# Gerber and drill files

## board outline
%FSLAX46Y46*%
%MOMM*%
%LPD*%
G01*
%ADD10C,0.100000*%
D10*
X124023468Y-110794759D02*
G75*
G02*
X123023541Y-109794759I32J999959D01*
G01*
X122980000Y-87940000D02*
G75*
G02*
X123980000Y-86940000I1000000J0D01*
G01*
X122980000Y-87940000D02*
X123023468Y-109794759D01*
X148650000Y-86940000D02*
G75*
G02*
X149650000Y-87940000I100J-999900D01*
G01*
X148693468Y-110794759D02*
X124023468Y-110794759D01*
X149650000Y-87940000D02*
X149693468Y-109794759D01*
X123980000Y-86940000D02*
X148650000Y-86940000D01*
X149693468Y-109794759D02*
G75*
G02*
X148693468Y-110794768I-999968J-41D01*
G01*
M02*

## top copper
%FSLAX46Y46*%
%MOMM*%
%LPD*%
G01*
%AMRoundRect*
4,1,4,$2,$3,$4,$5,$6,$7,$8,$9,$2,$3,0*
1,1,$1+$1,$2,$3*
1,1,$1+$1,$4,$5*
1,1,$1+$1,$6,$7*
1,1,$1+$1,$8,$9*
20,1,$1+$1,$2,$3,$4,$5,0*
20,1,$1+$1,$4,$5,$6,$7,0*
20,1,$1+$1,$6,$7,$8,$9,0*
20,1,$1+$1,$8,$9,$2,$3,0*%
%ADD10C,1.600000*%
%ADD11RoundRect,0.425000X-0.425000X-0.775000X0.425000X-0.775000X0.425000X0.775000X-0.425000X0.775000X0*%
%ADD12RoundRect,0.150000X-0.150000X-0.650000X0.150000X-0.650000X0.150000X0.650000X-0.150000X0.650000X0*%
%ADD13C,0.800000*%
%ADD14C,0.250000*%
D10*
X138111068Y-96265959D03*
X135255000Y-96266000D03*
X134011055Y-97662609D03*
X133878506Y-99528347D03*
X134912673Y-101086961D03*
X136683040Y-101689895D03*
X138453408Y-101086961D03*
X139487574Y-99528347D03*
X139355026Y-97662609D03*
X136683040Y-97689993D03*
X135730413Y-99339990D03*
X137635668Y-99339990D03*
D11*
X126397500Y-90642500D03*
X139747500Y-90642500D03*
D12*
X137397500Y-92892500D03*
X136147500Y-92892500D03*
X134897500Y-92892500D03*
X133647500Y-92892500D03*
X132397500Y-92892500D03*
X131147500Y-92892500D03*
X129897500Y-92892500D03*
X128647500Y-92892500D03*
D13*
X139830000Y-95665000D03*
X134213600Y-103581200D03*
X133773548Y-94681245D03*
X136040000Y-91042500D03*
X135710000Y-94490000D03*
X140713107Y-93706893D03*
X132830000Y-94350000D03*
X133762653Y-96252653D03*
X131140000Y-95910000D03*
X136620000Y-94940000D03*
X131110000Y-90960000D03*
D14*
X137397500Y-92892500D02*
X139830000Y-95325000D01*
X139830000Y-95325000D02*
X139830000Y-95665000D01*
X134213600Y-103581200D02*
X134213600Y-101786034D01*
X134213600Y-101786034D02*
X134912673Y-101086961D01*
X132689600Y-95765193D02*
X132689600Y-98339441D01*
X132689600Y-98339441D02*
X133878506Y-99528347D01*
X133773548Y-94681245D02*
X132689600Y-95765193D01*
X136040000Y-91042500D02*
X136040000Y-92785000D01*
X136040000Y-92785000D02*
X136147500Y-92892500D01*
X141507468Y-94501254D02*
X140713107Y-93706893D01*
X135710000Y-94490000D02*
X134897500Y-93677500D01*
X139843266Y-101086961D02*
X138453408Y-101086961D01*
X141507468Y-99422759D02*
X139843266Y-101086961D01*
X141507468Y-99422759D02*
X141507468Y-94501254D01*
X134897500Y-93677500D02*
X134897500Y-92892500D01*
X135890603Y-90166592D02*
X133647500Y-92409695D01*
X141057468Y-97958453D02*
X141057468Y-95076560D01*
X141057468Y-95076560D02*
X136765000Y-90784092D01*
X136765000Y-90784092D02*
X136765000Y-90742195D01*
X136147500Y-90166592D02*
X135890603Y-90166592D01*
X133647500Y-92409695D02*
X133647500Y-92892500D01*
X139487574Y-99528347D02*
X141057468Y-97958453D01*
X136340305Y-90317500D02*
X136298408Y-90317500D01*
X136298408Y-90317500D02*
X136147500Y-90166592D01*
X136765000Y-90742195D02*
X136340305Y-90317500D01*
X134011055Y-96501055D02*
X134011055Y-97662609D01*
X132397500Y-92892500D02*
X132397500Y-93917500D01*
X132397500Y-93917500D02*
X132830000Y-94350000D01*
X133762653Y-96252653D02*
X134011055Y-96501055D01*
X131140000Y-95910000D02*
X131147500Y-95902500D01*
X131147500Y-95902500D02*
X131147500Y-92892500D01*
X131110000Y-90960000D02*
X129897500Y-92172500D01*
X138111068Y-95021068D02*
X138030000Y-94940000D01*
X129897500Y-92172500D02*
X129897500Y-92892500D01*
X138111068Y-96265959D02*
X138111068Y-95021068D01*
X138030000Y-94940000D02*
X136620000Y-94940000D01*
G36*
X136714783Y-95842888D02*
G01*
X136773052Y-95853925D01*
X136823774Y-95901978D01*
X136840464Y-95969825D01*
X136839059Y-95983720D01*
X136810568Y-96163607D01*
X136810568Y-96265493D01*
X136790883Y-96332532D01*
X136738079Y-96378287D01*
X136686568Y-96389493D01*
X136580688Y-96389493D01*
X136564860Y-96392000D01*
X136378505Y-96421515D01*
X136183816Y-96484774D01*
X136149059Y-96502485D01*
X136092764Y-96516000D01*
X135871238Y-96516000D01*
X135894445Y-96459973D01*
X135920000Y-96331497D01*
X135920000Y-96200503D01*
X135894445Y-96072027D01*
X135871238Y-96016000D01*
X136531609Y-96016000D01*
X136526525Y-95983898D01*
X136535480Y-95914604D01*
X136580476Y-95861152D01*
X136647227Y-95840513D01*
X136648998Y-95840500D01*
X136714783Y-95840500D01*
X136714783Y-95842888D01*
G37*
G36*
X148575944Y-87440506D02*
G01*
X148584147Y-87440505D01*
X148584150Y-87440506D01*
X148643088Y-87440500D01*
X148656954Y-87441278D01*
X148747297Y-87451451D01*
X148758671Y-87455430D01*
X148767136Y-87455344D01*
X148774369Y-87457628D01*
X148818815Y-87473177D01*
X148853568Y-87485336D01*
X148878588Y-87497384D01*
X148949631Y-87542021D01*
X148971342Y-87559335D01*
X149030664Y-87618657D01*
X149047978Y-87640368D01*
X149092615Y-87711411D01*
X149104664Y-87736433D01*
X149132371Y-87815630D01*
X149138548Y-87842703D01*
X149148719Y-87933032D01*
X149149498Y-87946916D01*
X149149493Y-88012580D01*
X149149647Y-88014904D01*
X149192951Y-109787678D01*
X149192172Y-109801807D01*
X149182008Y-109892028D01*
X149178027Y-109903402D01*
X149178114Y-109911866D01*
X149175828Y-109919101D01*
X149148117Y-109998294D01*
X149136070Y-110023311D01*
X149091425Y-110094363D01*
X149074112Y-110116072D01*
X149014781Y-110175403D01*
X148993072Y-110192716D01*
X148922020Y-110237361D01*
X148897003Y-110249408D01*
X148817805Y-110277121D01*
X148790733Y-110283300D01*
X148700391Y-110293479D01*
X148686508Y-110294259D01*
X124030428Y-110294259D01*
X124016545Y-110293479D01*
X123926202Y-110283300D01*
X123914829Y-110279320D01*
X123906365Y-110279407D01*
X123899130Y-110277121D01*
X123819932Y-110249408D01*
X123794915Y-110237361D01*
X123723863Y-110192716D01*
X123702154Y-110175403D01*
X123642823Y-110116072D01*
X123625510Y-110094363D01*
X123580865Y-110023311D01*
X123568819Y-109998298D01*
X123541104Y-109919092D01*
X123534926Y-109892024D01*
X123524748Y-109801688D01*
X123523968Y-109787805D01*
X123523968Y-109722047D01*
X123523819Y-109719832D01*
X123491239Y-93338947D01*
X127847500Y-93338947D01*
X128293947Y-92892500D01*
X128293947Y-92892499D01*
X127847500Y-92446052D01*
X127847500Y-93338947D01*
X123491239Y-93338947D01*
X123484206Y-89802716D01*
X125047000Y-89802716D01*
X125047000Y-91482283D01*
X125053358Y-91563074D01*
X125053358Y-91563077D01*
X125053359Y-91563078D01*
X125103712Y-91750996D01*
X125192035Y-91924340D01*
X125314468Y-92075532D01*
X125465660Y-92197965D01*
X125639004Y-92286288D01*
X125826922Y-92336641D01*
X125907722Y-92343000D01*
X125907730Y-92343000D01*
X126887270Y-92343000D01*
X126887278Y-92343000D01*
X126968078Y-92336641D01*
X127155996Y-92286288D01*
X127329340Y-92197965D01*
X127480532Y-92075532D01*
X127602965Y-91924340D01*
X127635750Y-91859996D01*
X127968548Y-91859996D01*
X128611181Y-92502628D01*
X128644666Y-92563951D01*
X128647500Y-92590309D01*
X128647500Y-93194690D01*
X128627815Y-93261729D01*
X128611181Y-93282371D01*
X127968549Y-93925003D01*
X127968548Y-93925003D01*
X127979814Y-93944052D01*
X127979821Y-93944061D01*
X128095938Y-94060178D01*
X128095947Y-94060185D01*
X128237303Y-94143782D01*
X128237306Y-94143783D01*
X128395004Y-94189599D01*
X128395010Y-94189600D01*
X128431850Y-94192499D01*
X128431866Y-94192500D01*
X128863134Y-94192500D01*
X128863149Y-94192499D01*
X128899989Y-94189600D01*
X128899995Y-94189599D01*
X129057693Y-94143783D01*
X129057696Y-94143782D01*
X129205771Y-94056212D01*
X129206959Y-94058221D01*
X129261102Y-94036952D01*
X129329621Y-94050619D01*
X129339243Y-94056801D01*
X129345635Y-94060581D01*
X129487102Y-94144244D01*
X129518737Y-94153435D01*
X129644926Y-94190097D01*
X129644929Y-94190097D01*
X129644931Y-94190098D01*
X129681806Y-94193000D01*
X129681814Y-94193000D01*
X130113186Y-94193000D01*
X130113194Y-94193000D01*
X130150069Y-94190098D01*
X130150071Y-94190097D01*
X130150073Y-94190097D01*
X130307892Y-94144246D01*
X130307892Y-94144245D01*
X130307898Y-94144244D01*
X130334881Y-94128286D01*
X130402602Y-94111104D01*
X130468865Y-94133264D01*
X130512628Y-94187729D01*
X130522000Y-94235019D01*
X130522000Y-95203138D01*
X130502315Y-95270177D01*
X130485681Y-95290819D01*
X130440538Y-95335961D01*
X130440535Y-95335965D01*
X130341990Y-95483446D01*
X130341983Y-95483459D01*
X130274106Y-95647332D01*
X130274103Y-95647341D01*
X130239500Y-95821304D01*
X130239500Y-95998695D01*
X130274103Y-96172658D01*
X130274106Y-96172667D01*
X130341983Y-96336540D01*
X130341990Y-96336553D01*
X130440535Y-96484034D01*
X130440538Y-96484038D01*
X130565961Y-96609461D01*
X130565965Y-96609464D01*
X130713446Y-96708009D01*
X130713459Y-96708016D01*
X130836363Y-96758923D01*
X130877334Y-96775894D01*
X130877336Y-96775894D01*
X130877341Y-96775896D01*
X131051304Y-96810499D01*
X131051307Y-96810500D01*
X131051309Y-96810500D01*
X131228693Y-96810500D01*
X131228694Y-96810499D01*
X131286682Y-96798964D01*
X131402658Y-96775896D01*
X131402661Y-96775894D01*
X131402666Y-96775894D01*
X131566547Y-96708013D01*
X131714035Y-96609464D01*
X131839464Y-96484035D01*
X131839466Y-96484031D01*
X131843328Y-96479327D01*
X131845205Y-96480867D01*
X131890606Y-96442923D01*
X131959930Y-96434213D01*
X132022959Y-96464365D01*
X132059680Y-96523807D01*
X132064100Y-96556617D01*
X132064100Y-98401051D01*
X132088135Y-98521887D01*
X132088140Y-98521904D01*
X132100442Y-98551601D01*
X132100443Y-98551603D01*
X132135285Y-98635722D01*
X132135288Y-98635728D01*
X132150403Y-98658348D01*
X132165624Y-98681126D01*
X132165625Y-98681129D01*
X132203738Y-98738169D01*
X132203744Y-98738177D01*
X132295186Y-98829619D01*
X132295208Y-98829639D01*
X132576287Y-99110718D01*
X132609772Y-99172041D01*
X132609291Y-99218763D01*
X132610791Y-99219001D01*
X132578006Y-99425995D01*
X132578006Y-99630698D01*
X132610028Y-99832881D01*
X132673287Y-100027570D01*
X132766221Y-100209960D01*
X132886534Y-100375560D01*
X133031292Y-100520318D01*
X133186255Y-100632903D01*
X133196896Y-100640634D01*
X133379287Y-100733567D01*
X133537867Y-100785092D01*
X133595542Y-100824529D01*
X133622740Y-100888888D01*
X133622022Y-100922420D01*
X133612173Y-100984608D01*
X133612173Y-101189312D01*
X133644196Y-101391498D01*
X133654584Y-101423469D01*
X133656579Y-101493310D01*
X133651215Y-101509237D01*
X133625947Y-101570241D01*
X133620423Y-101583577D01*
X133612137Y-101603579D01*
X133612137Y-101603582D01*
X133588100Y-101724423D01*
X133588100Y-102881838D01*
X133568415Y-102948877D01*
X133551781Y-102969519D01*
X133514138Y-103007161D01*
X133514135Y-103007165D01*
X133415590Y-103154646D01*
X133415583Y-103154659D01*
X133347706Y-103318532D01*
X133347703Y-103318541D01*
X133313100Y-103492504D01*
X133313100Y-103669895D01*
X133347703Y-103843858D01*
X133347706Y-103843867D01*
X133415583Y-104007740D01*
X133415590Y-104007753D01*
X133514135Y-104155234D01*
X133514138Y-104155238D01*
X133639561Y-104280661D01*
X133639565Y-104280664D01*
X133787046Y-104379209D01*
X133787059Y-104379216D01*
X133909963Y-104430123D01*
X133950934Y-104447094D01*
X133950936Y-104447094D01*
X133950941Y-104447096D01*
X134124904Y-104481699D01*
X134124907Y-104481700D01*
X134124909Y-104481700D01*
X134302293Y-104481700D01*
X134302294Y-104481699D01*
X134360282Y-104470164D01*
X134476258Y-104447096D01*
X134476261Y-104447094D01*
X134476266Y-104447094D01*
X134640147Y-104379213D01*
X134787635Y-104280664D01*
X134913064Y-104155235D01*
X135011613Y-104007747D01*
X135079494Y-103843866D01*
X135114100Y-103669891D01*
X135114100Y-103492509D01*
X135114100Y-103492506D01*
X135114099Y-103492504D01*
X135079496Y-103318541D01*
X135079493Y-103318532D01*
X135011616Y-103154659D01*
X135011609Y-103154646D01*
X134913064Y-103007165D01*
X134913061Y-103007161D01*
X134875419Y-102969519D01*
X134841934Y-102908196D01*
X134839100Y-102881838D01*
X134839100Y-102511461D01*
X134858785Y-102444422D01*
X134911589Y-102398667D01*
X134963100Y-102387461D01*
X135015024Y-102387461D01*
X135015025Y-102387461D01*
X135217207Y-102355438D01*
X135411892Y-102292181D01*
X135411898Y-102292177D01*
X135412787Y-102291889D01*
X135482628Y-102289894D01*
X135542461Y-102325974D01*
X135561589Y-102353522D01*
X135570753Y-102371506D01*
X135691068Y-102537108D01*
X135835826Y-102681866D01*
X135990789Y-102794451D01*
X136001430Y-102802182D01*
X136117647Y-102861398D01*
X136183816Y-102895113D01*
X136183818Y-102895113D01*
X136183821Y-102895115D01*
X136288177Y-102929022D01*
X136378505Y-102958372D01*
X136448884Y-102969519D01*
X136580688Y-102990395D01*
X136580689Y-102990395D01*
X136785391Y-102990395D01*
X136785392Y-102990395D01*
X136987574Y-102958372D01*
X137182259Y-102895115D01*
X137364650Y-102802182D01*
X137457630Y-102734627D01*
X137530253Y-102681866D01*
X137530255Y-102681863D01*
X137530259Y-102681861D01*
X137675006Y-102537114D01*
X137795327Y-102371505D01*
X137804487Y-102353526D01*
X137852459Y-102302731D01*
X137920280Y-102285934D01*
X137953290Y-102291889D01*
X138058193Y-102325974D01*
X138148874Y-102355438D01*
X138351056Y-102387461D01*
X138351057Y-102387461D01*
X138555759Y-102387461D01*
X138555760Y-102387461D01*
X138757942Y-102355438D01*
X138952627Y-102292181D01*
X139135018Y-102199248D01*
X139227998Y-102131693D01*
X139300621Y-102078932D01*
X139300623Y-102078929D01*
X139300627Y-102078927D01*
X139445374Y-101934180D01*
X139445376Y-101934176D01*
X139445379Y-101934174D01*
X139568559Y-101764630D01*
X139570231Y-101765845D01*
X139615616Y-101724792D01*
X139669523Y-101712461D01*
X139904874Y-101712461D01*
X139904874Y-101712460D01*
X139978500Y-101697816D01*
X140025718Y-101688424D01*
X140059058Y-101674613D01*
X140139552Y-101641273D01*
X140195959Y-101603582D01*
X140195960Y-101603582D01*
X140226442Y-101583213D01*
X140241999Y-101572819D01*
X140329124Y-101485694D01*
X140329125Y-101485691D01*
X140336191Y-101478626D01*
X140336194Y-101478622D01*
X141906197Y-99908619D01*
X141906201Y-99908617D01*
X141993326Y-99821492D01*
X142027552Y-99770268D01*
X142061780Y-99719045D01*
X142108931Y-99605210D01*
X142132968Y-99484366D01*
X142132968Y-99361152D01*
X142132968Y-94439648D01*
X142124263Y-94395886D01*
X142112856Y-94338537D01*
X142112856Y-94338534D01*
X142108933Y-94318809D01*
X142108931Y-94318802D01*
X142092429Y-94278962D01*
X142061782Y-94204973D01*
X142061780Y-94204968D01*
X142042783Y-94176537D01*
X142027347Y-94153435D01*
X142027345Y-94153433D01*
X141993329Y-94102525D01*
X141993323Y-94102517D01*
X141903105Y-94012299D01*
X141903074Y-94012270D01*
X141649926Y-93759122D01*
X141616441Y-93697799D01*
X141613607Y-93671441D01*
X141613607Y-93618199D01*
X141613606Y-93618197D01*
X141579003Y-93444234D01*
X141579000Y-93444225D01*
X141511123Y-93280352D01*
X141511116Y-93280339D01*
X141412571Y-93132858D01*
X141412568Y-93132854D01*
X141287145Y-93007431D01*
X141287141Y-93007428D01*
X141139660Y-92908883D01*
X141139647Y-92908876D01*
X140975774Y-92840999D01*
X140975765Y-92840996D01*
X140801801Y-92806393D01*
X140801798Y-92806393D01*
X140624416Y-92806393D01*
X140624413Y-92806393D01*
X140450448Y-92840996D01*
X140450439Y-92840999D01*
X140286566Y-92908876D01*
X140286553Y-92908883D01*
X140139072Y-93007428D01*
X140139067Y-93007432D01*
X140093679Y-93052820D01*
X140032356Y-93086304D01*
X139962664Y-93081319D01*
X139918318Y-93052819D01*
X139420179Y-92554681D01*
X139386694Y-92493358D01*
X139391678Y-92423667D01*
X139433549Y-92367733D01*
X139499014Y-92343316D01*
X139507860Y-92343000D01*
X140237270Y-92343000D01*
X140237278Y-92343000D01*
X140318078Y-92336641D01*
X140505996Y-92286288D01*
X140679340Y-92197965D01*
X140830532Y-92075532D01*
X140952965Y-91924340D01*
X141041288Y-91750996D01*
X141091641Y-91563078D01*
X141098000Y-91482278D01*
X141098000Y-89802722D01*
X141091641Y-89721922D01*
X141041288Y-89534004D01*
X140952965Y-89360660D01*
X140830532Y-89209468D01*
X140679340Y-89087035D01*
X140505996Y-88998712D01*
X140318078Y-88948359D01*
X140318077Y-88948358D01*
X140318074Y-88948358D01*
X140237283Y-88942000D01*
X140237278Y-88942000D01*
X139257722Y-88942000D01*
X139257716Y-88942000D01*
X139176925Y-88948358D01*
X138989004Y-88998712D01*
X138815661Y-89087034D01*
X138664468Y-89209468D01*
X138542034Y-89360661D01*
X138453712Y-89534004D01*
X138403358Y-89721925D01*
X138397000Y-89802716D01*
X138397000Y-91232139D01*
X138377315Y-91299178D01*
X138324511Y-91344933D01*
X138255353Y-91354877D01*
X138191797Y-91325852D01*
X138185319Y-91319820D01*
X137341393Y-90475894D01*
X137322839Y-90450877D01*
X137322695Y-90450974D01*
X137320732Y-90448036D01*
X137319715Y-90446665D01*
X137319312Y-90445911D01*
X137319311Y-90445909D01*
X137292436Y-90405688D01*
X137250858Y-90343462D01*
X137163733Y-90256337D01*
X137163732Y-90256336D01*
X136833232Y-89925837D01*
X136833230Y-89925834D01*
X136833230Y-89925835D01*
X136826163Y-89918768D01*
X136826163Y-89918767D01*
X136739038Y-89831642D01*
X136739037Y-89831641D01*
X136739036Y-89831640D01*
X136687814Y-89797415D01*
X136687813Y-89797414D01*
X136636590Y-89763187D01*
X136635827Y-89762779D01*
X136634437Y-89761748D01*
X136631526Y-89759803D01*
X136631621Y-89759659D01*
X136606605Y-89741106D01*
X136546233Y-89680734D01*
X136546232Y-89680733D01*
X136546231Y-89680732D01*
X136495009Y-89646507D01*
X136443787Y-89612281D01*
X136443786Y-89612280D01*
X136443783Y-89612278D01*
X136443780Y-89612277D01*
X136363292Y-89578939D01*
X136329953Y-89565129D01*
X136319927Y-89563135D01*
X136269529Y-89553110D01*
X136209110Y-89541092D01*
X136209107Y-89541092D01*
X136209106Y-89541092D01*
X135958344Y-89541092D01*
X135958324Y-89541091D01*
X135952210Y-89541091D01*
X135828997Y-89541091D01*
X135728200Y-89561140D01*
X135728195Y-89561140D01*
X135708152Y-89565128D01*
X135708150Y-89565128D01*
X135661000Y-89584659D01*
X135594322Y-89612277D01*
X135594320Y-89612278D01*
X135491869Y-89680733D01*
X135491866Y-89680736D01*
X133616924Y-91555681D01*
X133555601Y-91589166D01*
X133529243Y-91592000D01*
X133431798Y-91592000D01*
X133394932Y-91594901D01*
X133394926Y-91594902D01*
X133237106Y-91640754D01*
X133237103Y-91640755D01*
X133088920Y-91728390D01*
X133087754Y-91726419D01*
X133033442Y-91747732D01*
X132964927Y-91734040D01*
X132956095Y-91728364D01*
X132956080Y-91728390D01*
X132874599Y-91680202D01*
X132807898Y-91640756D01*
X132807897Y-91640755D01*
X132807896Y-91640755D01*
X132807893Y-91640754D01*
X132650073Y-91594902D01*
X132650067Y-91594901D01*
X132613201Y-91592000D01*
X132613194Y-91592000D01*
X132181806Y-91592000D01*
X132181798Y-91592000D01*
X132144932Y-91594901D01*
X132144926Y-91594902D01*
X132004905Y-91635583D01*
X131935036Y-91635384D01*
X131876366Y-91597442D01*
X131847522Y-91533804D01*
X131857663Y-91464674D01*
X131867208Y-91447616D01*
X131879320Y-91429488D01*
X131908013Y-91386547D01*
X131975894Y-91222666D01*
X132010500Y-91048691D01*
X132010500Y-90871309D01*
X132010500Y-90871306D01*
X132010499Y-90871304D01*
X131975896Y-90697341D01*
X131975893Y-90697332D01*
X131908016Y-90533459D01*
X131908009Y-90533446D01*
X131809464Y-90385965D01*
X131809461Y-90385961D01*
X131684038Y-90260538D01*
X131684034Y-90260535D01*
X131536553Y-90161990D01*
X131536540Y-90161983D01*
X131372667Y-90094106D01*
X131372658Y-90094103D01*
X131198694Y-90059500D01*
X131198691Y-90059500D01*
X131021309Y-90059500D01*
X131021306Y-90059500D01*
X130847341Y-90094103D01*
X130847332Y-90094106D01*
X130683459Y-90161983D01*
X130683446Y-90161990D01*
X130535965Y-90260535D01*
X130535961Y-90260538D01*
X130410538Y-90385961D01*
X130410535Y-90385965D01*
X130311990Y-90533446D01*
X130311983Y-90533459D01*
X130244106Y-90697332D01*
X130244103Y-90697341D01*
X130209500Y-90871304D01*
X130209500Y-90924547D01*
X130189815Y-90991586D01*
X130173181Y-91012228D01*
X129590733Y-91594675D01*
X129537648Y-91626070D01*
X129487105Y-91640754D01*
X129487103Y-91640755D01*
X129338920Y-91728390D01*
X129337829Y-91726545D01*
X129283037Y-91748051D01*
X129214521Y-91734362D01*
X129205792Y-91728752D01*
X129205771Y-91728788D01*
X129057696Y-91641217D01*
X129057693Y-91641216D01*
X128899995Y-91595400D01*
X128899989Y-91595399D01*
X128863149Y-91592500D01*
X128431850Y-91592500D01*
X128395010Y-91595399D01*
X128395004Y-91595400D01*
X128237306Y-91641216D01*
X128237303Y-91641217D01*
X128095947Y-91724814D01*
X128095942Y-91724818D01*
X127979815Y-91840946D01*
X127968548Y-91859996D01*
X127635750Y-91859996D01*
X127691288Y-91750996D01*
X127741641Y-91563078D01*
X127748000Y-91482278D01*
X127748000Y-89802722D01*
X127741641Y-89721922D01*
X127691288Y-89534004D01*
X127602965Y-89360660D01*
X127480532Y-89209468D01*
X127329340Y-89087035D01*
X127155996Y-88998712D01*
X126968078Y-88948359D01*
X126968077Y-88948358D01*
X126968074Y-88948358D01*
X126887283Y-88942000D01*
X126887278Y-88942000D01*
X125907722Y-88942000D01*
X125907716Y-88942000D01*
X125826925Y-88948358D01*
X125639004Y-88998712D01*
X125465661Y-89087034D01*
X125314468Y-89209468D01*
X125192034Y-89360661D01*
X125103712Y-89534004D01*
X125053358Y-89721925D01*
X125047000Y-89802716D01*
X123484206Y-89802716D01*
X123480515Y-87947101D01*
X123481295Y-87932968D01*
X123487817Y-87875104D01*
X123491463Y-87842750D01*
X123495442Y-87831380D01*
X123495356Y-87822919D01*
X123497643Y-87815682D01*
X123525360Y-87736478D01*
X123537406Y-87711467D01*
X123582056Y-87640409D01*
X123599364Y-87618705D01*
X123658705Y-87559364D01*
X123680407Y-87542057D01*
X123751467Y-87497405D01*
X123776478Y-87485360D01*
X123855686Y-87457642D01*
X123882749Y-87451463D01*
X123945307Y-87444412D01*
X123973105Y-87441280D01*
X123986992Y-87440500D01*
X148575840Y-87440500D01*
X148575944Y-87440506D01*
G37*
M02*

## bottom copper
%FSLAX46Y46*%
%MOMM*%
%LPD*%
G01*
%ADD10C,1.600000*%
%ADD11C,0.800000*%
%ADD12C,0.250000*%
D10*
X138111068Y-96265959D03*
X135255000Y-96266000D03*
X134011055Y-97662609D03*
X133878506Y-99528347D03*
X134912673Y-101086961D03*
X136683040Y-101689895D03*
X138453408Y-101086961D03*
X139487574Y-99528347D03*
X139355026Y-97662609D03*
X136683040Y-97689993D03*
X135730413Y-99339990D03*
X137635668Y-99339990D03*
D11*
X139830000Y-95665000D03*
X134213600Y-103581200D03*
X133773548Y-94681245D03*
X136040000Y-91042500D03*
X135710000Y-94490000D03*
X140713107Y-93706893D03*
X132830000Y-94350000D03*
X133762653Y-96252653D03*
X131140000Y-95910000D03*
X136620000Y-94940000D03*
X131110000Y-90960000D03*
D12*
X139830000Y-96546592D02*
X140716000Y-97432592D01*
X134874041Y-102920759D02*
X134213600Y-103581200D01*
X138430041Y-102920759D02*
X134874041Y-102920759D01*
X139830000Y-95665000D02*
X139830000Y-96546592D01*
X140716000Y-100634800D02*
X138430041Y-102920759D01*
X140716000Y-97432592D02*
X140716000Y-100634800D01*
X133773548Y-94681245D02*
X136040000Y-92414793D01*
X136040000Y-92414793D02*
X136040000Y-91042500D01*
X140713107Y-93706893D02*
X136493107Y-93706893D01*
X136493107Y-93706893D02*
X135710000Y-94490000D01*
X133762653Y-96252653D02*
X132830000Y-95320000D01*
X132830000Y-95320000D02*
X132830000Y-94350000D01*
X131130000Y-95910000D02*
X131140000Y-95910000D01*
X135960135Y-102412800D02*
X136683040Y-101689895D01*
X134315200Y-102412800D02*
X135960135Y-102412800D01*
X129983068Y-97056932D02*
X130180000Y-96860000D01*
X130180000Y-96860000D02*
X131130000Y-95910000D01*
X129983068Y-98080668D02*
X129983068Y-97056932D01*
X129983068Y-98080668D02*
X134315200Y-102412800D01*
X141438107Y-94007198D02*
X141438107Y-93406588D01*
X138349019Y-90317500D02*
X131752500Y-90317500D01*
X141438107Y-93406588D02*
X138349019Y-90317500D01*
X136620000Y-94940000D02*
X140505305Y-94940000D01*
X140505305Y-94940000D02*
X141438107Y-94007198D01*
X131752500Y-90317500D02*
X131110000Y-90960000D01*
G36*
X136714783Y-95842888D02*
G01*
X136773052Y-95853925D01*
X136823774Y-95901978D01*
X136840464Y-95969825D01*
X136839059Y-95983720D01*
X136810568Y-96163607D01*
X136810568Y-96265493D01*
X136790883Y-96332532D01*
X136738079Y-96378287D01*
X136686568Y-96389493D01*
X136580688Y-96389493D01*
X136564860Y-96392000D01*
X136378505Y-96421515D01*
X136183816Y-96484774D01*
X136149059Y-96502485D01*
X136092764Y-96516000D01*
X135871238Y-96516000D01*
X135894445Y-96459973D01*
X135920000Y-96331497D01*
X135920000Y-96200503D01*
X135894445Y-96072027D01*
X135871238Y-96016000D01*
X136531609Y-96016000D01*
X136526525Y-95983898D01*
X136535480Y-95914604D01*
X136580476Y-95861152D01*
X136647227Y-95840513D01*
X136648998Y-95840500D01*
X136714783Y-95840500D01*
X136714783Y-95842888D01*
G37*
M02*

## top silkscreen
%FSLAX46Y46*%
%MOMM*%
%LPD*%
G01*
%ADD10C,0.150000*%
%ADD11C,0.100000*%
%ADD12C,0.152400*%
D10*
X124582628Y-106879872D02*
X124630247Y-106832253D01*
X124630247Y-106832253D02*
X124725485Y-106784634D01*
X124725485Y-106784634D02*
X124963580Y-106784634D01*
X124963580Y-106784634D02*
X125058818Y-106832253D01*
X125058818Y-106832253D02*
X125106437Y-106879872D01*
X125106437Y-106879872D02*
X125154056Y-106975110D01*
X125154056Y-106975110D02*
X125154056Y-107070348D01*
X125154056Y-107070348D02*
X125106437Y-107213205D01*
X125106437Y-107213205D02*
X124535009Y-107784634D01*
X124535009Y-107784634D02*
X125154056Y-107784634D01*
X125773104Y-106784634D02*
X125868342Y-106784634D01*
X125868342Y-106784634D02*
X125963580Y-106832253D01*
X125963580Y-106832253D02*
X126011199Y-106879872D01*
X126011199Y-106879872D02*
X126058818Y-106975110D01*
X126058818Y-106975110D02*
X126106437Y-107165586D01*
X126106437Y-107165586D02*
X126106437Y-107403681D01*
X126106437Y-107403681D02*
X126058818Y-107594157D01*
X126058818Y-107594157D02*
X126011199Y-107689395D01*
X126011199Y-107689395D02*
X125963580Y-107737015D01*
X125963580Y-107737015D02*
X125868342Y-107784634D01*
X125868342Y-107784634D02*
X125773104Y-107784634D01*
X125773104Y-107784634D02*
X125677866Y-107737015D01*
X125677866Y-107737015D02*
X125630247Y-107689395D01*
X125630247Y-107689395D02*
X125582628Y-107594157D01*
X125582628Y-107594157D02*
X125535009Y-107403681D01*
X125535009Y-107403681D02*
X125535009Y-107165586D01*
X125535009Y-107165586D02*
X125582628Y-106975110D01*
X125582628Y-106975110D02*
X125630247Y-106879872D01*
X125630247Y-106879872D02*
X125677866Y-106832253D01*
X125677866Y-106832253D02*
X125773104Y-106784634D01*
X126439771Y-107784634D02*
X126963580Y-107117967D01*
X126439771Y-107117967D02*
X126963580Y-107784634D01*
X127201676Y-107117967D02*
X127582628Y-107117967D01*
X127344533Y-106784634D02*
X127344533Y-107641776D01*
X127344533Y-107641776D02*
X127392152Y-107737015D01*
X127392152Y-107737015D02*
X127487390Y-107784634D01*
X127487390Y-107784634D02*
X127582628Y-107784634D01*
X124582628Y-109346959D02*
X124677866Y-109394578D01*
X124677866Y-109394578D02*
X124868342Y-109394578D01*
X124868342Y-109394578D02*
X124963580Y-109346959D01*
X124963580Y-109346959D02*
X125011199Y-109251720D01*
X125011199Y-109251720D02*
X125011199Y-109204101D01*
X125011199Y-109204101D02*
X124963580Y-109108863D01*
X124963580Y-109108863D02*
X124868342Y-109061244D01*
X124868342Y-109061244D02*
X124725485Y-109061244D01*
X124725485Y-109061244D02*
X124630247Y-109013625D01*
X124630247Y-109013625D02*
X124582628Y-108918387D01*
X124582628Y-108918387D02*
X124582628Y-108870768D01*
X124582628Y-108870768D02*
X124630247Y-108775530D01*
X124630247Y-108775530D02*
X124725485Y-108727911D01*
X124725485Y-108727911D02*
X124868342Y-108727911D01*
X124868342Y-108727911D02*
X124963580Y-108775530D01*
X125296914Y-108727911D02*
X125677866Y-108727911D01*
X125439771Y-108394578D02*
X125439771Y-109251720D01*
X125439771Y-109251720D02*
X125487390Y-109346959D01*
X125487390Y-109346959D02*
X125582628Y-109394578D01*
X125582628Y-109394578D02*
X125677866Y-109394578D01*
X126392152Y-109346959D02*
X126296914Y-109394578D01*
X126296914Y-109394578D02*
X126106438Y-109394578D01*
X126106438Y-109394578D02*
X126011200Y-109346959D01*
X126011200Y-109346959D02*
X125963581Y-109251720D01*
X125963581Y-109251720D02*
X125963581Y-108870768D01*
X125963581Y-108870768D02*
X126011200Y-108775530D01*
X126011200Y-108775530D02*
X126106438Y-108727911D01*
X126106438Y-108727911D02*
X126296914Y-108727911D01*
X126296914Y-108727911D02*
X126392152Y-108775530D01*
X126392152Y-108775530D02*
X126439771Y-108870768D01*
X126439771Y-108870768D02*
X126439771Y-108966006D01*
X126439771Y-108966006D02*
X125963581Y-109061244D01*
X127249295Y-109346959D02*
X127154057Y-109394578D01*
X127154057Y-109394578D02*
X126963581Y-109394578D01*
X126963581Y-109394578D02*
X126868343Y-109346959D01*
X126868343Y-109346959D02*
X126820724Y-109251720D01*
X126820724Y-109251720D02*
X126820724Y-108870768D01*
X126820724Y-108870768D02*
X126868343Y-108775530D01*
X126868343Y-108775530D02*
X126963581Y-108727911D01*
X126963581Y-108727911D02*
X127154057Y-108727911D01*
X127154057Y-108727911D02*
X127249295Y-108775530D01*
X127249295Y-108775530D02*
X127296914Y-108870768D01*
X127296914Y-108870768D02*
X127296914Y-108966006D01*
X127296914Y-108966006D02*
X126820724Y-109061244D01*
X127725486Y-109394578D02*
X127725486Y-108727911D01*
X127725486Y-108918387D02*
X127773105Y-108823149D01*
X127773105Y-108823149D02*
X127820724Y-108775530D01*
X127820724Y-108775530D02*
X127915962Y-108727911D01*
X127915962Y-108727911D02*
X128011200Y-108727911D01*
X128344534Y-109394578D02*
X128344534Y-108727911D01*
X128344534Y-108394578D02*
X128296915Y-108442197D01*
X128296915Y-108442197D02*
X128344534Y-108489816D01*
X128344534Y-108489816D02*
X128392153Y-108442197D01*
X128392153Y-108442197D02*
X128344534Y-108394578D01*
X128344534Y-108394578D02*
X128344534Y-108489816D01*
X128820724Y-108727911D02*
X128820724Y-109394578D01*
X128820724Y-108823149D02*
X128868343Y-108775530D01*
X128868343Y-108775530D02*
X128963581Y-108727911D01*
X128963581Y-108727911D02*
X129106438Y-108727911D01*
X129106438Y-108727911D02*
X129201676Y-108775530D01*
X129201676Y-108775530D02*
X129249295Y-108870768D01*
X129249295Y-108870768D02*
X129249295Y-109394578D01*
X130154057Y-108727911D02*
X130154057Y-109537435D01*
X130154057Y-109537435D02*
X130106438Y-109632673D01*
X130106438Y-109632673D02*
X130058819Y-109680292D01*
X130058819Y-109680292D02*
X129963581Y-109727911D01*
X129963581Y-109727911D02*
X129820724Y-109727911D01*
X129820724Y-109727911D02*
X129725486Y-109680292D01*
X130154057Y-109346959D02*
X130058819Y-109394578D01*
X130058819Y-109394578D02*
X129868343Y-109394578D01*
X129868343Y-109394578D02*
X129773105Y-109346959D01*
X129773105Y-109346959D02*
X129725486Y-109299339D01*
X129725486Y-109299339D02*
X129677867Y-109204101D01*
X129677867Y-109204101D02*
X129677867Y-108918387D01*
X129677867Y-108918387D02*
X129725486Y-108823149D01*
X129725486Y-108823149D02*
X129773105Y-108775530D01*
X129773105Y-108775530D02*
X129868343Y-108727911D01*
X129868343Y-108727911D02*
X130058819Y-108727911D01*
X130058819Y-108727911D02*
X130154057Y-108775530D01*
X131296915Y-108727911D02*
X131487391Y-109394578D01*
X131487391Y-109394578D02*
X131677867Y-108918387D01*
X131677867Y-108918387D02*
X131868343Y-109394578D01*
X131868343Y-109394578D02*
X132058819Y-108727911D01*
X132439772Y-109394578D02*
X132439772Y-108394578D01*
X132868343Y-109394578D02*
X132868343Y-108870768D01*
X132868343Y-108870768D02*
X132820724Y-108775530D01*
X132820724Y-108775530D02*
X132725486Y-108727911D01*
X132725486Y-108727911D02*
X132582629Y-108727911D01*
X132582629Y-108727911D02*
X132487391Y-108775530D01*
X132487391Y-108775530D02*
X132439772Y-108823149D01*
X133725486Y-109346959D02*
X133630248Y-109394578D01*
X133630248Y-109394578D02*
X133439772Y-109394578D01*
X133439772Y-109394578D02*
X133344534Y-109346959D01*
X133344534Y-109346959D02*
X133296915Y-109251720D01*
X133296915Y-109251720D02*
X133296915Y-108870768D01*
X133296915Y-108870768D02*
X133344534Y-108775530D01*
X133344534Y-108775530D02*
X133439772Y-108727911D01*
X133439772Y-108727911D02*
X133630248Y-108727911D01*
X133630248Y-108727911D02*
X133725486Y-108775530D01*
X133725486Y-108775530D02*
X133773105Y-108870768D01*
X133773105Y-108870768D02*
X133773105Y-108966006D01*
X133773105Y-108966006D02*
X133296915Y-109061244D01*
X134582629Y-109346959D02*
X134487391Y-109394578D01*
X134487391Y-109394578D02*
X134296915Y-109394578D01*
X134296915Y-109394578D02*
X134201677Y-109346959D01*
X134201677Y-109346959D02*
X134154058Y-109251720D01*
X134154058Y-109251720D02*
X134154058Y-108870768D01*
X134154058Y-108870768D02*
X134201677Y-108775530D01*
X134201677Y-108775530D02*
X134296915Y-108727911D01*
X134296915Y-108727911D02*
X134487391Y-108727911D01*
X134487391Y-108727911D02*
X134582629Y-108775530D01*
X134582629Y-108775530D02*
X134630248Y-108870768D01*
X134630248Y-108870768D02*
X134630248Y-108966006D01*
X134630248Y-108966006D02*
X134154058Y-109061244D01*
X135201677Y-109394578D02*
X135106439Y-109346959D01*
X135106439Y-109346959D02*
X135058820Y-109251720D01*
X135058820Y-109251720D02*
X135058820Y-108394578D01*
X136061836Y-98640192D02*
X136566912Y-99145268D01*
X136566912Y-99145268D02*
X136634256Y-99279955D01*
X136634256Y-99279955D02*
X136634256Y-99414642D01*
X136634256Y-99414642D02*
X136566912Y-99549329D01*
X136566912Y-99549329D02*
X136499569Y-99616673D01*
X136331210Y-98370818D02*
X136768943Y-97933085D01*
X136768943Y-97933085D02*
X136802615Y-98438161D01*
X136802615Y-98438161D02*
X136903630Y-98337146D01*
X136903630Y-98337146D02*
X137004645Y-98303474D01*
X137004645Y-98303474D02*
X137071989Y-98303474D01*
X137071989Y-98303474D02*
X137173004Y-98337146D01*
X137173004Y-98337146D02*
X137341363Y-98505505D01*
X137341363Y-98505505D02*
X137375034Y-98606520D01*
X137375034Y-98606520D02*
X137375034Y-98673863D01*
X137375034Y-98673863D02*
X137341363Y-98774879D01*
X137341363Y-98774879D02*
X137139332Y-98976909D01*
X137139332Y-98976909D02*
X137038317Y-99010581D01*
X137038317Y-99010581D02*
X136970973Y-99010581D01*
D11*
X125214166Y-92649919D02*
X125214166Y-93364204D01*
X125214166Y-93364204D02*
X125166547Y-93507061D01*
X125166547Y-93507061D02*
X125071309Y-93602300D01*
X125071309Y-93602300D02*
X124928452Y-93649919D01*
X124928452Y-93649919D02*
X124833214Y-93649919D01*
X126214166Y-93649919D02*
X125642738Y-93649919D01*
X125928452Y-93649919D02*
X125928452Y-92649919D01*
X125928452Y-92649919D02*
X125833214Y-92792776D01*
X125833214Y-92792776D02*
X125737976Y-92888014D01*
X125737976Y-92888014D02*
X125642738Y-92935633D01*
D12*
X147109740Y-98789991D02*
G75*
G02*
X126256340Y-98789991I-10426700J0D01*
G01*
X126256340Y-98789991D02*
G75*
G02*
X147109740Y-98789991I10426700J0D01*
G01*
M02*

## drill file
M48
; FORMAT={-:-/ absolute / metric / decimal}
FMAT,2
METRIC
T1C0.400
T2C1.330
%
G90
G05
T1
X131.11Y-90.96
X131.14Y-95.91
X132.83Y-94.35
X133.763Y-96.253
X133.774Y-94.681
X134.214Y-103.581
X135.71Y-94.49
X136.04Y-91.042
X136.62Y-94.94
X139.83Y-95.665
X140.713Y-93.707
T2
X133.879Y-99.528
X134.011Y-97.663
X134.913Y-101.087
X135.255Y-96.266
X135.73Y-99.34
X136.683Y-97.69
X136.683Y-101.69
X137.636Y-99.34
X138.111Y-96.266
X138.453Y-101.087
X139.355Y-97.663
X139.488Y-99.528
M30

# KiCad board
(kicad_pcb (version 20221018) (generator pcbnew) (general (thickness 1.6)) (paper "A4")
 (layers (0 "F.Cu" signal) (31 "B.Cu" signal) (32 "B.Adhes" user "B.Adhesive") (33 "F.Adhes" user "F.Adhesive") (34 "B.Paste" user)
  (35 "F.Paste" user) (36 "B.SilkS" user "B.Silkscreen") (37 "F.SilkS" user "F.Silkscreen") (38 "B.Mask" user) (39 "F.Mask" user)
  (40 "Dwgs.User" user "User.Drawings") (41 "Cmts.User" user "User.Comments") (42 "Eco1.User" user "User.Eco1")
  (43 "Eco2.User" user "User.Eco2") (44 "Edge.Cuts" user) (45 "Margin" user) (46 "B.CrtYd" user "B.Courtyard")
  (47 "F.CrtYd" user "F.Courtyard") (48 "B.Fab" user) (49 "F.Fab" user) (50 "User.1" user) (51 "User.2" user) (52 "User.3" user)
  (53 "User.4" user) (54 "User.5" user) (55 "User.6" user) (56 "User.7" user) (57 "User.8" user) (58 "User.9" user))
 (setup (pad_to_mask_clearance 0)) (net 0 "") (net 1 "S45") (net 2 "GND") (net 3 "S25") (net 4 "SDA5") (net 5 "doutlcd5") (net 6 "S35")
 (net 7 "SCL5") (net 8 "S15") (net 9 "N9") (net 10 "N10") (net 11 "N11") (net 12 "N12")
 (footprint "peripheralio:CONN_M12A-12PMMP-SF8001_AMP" (layer "F.Cu") (at 138.111068 96.265959 45)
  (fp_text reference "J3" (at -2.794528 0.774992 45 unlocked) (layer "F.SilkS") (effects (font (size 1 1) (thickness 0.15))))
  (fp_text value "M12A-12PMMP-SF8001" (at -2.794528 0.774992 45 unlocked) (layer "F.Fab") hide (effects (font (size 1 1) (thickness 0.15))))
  (fp_circle (center -2.794528 0.774992) (end 7.632172 0.774992) (stroke (width 0.1524) (type solid)) (fill none) (layer "F.SilkS"))
  (pad "1" thru_hole circle (at 0 0 45) (size 1.6 1.6) (drill 1.33) (layers "*.Cu" "*.Mask") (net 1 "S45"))
  (pad "2" thru_hole circle (at -2.019574 -2.019516 45) (size 1.6 1.6) (drill 1.33) (layers "*.Cu" "*.Mask") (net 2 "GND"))
  (pad "3" thru_hole circle (at -3.886728 -1.911566 135) (size 1.6 1.6) (drill 1.33) (layers "*.Cu" "*.Mask") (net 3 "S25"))
  (pad "4" thru_hole circle (at -5.29973 -0.686016 45) (size 1.6 1.6) (drill 1.33) (layers "*.Cu" "*.Mask") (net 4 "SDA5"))
  (pad "5" thru_hole circle (at -5.67057 1.147356 45) (size 1.6 1.6) (drill 1.33) (layers "*.Cu" "*.Mask") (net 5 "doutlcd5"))
  (pad "6" thru_hole circle (at -4.84507 2.825534 45) (size 1.6 1.6) (drill 1.33) (layers "*.Cu" "*.Mask") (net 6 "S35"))
  (pad "7" thru_hole circle (at -3.166892 3.651034 45) (size 1.6 1.6) (drill 1.33) (layers "*.Cu" "*.Mask") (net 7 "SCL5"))
  (pad "8" thru_hole circle (at -1.33352 3.280194 45) (size 1.6 1.6) (drill 1.33) (layers "*.Cu" "*.Mask") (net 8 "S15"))
  (pad "9" thru_hole circle (at -0.10797 1.867192 45) (size 1.6 1.6) (drill 1.33) (layers "*.Cu" "*.Mask") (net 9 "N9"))
  (pad "10" thru_hole circle (at -2.016712 -0.002824 45) (size 1.6 1.6) (drill 1.33) (layers "*.Cu" "*.Mask") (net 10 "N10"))
  (pad "11" thru_hole circle (at -3.857046 0.490291 255) (size 1.6 1.6) (drill 1.33) (layers "*.Cu" "*.Mask") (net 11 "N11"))
  (pad "12" thru_hole circle (at -2.509827 1.83751 285) (size 1.6 1.6) (drill 1.33) (layers "*.Cu" "*.Mask") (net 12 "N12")))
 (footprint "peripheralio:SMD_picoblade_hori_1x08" (layer "F.Cu") (at 125.5475 93.6925)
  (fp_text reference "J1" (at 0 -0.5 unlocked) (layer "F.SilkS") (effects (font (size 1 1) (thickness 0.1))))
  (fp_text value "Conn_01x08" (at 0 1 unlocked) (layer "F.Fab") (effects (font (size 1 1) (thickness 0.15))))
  (pad "" smd roundrect (at 0.85 -3.05) (size 1.7 2.4) (layers "F.Cu" "F.Paste" "F.Mask") (roundrect_rratio 0.25) (thermal_bridge_angle 45))
  (pad "" smd roundrect (at 14.2 -3.05) (size 1.7 2.4) (layers "F.Cu" "F.Paste" "F.Mask") (roundrect_rratio 0.25) (thermal_bridge_angle 45))
  (pad "1" smd roundrect (at 11.85 -0.8) (size 0.6 1.6) (layers "F.Cu" "F.Paste" "F.Mask") (roundrect_rratio 0.25) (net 5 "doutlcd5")
   (thermal_bridge_angle 45))
  (pad "2" smd roundrect (at 10.6 -0.8) (size 0.6 1.6) (layers "F.Cu" "F.Paste" "F.Mask") (roundrect_rratio 0.25) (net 4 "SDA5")
   (thermal_bridge_angle 45))
  (pad "3" smd roundrect (at 9.35 -0.8) (size 0.6 1.6) (layers "F.Cu" "F.Paste" "F.Mask") (roundrect_rratio 0.25) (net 7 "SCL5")
   (thermal_bridge_angle 45))
  (pad "4" smd roundrect (at 8.1 -0.8) (size 0.6 1.6) (layers "F.Cu" "F.Paste" "F.Mask") (roundrect_rratio 0.25) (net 8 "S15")
   (thermal_bridge_angle 45))
  (pad "5" smd roundrect (at 6.85 -0.8) (size 0.6 1.6) (layers "F.Cu" "F.Paste" "F.Mask") (roundrect_rratio 0.25) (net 3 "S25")
   (thermal_bridge_angle 45))
  (pad "6" smd roundrect (at 5.6 -0.8) (size 0.6 1.6) (layers "F.Cu" "F.Paste" "F.Mask") (roundrect_rratio 0.25) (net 6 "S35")
   (thermal_bridge_angle 45))
  (pad "7" smd roundrect (at 4.35 -0.8) (size 0.6 1.6) (layers "F.Cu" "F.Paste" "F.Mask") (roundrect_rratio 0.25) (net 1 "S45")
   (thermal_bridge_angle 45))
  (pad "8" smd roundrect (at 3.1 -0.8) (size 0.6 1.6) (layers "F.Cu" "F.Paste" "F.Mask") (roundrect_rratio 0.25) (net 2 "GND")
   (thermal_bridge_angle 45)))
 (gr_arc (start 124.023468 110.794759) (mid 123.316361 110.501866) (end 123.023468 109.794759) (stroke (width 0.1) (type default))
  (layer "Edge.Cuts"))
 (gr_arc (start 122.98 87.94) (mid 123.272906 87.232908) (end 123.98 86.94) (stroke (width 0.1) (type default)) (layer "Edge.Cuts"))
 (gr_line (start 122.98 87.94) (end 123.023468 109.794759) (stroke (width 0.1) (type default)) (layer "Edge.Cuts"))
 (gr_arc (start 148.65 86.94) (mid 149.357142 87.232879) (end 149.65 87.94) (stroke (width 0.1) (type default)) (layer "Edge.Cuts"))
 (gr_line (start 148.693468 110.794759) (end 124.023468 110.794759) (stroke (width 0.1) (type default)) (layer "Edge.Cuts"))
 (gr_line (start 149.65 87.94) (end 149.693468 109.794759) (stroke (width 0.1) (type default)) (layer "Edge.Cuts"))
 (gr_line (start 123.98 86.94) (end 148.65 86.94) (stroke (width 0.1) (type default)) (layer "Edge.Cuts"))
 (gr_arc (start 149.693468 109.794759) (mid 149.400575 110.501866) (end 148.693468 110.794759) (stroke (width 0.1) (type default))
  (layer "Edge.Cuts"))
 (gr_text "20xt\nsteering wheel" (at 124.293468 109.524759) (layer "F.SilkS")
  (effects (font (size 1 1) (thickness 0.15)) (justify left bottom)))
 (segment (start 137.3975 92.8925) (end 139.83 95.325) (width 0.25) (layer "F.Cu") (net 5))
 (segment (start 139.83 95.325) (end 139.83 95.665) (width 0.25) (layer "F.Cu") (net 5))
 (segment (start 134.2136 103.5812) (end 134.2136 101.786034) (width 0.25) (layer "F.Cu") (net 5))
 (segment (start 134.2136 101.786034) (end 134.912673 101.086961) (width 0.25) (layer "F.Cu") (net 5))
 (via (at 139.83 95.665) (size 0.8) (drill 0.4) (layers "F.Cu" "B.Cu") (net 5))
 (via (at 134.2136 103.5812) (size 0.8) (drill 0.4) (layers "F.Cu" "B.Cu") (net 5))
 (segment (start 139.83 96.546592) (end 140.716 97.432592) (width 0.25) (layer "B.Cu") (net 5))
 (segment (start 134.874041 102.920759) (end 134.2136 103.5812) (width 0.25) (layer "B.Cu") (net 5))
 (segment (start 138.430041 102.920759) (end 134.874041 102.920759) (width 0.25) (layer "B.Cu") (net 5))
 (segment (start 139.83 95.665) (end 139.83 96.546592) (width 0.25) (layer "B.Cu") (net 5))
 (segment (start 140.716 100.6348) (end 138.430041 102.920759) (width 0.25) (layer "B.Cu") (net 5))
 (segment (start 140.716 97.432592) (end 140.716 100.6348) (width 0.25) (layer "B.Cu") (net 5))
 (segment (start 132.6896 95.765193) (end 132.6896 98.339441) (width 0.25) (layer "F.Cu") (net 4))
 (segment (start 132.6896 98.339441) (end 133.878506 99.528347) (width 0.25) (layer "F.Cu") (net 4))
 (segment (start 133.773548 94.681245) (end 132.6896 95.765193) (width 0.25) (layer "F.Cu") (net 4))
 (segment (start 136.04 91.0425) (end 136.04 92.785) (width 0.25) (layer "F.Cu") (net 4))
 (segment (start 136.04 92.785) (end 136.1475 92.8925) (width 0.25) (layer "F.Cu") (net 4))
 (via (at 133.773548 94.681245) (size 0.8) (drill 0.4) (layers "F.Cu" "B.Cu") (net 4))
 (via (at 136.04 91.0425) (size 0.8) (drill 0.4) (layers "F.Cu" "B.Cu") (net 4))
 (segment (start 133.773548 94.681245) (end 136.04 92.414793) (width 0.25) (layer "B.Cu") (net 4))
 (segment (start 136.04 92.414793) (end 136.04 91.0425) (width 0.25) (layer "B.Cu") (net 4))
 (segment (start 141.507468 94.501254) (end 140.713107 93.706893) (width 0.25) (layer "F.Cu") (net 7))
 (segment (start 135.71 94.49) (end 134.8975 93.6775) (width 0.25) (layer "F.Cu") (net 7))
 (segment (start 139.843266 101.086961) (end 138.453408 101.086961) (width 0.25) (layer "F.Cu") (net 7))
 (segment (start 141.507468 99.422759) (end 139.843266 101.086961) (width 0.25) (layer "F.Cu") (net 7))
 (segment (start 141.507468 99.422759) (end 141.507468 94.501254) (width 0.25) (layer "F.Cu") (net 7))
 (segment (start 134.8975 93.6775) (end 134.8975 92.8925) (width 0.25) (layer "F.Cu") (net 7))
 (via (at 135.71 94.49) (size 0.8) (drill 0.4) (layers "F.Cu" "B.Cu") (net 7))
 (via (at 140.713107 93.706893) (size 0.8) (drill 0.4) (layers "F.Cu" "B.Cu") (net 7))
 (segment (start 140.713107 93.706893) (end 136.493107 93.706893) (width 0.25) (layer "B.Cu") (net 7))
 (segment (start 136.493107 93.706893) (end 135.71 94.49) (width 0.25) (layer "B.Cu") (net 7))
 (segment (start 135.890603 90.166592) (end 133.6475 92.409695) (width 0.25) (layer "F.Cu") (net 8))
 (segment (start 141.057468 97.958453) (end 141.057468 95.07656) (width 0.25) (layer "F.Cu") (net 8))
 (segment (start 141.057468 95.07656) (end 136.765 90.784092) (width 0.25) (layer "F.Cu") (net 8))
 (segment (start 136.765 90.784092) (end 136.765 90.742195) (width 0.25) (layer "F.Cu") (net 8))
 (segment (start 136.1475 90.166592) (end 135.890603 90.166592) (width 0.25) (layer "F.Cu") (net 8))
 (segment (start 133.6475 92.409695) (end 133.6475 92.8925) (width 0.25) (layer "F.Cu") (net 8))
 (segment (start 139.487574 99.528347) (end 141.057468 97.958453) (width 0.25) (layer "F.Cu") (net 8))
 (segment (start 136.340305 90.3175) (end 136.298408 90.3175) (width 0.25) (layer "F.Cu") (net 8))
 (segment (start 136.298408 90.3175) (end 136.1475 90.166592) (width 0.25) (layer "F.Cu") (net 8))
 (segment (start 136.765 90.742195) (end 136.340305 90.3175) (width 0.25) (layer "F.Cu") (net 8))
 (segment (start 134.011055 96.501055) (end 134.011055 97.662609) (width 0.25) (layer "F.Cu") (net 3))
 (segment (start 132.3975 92.8925) (end 132.3975 93.9175) (width 0.25) (layer "F.Cu") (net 3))
 (segment (start 132.3975 93.9175) (end 132.83 94.35) (width 0.25) (layer "F.Cu") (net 3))
 (segment (start 133.762653 96.252653) (end 134.011055 96.501055) (width 0.25) (layer "F.Cu") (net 3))
 (via (at 132.83 94.35) (size 0.8) (drill 0.4) (layers "F.Cu" "B.Cu") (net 3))
 (via (at 133.762653 96.252653) (size 0.8) (drill 0.4) (layers "F.Cu" "B.Cu") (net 3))
 (segment (start 133.762653 96.252653) (end 132.83 95.32) (width 0.25) (layer "B.Cu") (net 3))
 (segment (start 132.83 95.32) (end 132.83 94.35) (width 0.25) (layer "B.Cu") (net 3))
 (segment (start 131.14 95.91) (end 131.1475 95.9025) (width 0.25) (layer "F.Cu") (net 6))
 (segment (start 131.1475 95.9025) (end 131.1475 92.8925) (width 0.25) (layer "F.Cu") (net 6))
 (via (at 131.14 95.91) (size 0.8) (drill 0.4) (layers "F.Cu" "B.Cu") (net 6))
 (segment (start 131.13 95.91) (end 131.14 95.91) (width 0.25) (layer "B.Cu") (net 6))
 (segment (start 135.960135 102.4128) (end 136.68304 101.689895) (width 0.25) (layer "B.Cu") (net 6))
 (segment (start 134.3152 102.4128) (end 135.960135 102.4128) (width 0.25) (layer "B.Cu") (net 6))
 (segment (start 129.983068 97.056932) (end 130.18 96.86) (width 0.25) (layer "B.Cu") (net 6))
 (segment (start 130.18 96.86) (end 131.13 95.91) (width 0.25) (layer "B.Cu") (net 6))
 (segment (start 129.983068 98.080668) (end 129.983068 97.056932) (width 0.25) (layer "B.Cu") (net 6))
 (segment (start 129.983068 98.080668) (end 134.3152 102.4128) (width 0.25) (layer "B.Cu") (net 6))
 (segment (start 131.11 90.96) (end 129.8975 92.1725) (width 0.25) (layer "F.Cu") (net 1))
 (segment (start 138.111068 95.021068) (end 138.03 94.94) (width 0.25) (layer "F.Cu") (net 1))
 (segment (start 129.8975 92.1725) (end 129.8975 92.8925) (width 0.25) (layer "F.Cu") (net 1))
 (segment (start 138.111068 96.265959) (end 138.111068 95.021068) (width 0.25) (layer "F.Cu") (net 1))
 (segment (start 138.03 94.94) (end 136.62 94.94) (width 0.25) (layer "F.Cu") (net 1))
 (via (at 136.62 94.94) (size 0.8) (drill 0.4) (layers "F.Cu" "B.Cu") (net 1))
 (via (at 131.11 90.96) (size 0.8) (drill 0.4) (layers "F.Cu" "B.Cu") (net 1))
 (segment (start 141.438107 94.007198) (end 141.438107 93.406588) (width 0.25) (layer "B.Cu") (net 1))
 (segment (start 138.349019 90.3175) (end 131.7525 90.3175) (width 0.25) (layer "B.Cu") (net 1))
 (segment (start 141.438107 93.406588) (end 138.349019 90.3175) (width 0.25) (layer "B.Cu") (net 1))
 (segment (start 136.62 94.94) (end 140.505305 94.94) (width 0.25) (layer "B.Cu") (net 1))
 (segment (start 140.505305 94.94) (end 141.438107 94.007198) (width 0.25) (layer "B.Cu") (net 1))
 (segment (start 131.7525 90.3175) (end 131.11 90.96) (width 0.25) (layer "B.Cu") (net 1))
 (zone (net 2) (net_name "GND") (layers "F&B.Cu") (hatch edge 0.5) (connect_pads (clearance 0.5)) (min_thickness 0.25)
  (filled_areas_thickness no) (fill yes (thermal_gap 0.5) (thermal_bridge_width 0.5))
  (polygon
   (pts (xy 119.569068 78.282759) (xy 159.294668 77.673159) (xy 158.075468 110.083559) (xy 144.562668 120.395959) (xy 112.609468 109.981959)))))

